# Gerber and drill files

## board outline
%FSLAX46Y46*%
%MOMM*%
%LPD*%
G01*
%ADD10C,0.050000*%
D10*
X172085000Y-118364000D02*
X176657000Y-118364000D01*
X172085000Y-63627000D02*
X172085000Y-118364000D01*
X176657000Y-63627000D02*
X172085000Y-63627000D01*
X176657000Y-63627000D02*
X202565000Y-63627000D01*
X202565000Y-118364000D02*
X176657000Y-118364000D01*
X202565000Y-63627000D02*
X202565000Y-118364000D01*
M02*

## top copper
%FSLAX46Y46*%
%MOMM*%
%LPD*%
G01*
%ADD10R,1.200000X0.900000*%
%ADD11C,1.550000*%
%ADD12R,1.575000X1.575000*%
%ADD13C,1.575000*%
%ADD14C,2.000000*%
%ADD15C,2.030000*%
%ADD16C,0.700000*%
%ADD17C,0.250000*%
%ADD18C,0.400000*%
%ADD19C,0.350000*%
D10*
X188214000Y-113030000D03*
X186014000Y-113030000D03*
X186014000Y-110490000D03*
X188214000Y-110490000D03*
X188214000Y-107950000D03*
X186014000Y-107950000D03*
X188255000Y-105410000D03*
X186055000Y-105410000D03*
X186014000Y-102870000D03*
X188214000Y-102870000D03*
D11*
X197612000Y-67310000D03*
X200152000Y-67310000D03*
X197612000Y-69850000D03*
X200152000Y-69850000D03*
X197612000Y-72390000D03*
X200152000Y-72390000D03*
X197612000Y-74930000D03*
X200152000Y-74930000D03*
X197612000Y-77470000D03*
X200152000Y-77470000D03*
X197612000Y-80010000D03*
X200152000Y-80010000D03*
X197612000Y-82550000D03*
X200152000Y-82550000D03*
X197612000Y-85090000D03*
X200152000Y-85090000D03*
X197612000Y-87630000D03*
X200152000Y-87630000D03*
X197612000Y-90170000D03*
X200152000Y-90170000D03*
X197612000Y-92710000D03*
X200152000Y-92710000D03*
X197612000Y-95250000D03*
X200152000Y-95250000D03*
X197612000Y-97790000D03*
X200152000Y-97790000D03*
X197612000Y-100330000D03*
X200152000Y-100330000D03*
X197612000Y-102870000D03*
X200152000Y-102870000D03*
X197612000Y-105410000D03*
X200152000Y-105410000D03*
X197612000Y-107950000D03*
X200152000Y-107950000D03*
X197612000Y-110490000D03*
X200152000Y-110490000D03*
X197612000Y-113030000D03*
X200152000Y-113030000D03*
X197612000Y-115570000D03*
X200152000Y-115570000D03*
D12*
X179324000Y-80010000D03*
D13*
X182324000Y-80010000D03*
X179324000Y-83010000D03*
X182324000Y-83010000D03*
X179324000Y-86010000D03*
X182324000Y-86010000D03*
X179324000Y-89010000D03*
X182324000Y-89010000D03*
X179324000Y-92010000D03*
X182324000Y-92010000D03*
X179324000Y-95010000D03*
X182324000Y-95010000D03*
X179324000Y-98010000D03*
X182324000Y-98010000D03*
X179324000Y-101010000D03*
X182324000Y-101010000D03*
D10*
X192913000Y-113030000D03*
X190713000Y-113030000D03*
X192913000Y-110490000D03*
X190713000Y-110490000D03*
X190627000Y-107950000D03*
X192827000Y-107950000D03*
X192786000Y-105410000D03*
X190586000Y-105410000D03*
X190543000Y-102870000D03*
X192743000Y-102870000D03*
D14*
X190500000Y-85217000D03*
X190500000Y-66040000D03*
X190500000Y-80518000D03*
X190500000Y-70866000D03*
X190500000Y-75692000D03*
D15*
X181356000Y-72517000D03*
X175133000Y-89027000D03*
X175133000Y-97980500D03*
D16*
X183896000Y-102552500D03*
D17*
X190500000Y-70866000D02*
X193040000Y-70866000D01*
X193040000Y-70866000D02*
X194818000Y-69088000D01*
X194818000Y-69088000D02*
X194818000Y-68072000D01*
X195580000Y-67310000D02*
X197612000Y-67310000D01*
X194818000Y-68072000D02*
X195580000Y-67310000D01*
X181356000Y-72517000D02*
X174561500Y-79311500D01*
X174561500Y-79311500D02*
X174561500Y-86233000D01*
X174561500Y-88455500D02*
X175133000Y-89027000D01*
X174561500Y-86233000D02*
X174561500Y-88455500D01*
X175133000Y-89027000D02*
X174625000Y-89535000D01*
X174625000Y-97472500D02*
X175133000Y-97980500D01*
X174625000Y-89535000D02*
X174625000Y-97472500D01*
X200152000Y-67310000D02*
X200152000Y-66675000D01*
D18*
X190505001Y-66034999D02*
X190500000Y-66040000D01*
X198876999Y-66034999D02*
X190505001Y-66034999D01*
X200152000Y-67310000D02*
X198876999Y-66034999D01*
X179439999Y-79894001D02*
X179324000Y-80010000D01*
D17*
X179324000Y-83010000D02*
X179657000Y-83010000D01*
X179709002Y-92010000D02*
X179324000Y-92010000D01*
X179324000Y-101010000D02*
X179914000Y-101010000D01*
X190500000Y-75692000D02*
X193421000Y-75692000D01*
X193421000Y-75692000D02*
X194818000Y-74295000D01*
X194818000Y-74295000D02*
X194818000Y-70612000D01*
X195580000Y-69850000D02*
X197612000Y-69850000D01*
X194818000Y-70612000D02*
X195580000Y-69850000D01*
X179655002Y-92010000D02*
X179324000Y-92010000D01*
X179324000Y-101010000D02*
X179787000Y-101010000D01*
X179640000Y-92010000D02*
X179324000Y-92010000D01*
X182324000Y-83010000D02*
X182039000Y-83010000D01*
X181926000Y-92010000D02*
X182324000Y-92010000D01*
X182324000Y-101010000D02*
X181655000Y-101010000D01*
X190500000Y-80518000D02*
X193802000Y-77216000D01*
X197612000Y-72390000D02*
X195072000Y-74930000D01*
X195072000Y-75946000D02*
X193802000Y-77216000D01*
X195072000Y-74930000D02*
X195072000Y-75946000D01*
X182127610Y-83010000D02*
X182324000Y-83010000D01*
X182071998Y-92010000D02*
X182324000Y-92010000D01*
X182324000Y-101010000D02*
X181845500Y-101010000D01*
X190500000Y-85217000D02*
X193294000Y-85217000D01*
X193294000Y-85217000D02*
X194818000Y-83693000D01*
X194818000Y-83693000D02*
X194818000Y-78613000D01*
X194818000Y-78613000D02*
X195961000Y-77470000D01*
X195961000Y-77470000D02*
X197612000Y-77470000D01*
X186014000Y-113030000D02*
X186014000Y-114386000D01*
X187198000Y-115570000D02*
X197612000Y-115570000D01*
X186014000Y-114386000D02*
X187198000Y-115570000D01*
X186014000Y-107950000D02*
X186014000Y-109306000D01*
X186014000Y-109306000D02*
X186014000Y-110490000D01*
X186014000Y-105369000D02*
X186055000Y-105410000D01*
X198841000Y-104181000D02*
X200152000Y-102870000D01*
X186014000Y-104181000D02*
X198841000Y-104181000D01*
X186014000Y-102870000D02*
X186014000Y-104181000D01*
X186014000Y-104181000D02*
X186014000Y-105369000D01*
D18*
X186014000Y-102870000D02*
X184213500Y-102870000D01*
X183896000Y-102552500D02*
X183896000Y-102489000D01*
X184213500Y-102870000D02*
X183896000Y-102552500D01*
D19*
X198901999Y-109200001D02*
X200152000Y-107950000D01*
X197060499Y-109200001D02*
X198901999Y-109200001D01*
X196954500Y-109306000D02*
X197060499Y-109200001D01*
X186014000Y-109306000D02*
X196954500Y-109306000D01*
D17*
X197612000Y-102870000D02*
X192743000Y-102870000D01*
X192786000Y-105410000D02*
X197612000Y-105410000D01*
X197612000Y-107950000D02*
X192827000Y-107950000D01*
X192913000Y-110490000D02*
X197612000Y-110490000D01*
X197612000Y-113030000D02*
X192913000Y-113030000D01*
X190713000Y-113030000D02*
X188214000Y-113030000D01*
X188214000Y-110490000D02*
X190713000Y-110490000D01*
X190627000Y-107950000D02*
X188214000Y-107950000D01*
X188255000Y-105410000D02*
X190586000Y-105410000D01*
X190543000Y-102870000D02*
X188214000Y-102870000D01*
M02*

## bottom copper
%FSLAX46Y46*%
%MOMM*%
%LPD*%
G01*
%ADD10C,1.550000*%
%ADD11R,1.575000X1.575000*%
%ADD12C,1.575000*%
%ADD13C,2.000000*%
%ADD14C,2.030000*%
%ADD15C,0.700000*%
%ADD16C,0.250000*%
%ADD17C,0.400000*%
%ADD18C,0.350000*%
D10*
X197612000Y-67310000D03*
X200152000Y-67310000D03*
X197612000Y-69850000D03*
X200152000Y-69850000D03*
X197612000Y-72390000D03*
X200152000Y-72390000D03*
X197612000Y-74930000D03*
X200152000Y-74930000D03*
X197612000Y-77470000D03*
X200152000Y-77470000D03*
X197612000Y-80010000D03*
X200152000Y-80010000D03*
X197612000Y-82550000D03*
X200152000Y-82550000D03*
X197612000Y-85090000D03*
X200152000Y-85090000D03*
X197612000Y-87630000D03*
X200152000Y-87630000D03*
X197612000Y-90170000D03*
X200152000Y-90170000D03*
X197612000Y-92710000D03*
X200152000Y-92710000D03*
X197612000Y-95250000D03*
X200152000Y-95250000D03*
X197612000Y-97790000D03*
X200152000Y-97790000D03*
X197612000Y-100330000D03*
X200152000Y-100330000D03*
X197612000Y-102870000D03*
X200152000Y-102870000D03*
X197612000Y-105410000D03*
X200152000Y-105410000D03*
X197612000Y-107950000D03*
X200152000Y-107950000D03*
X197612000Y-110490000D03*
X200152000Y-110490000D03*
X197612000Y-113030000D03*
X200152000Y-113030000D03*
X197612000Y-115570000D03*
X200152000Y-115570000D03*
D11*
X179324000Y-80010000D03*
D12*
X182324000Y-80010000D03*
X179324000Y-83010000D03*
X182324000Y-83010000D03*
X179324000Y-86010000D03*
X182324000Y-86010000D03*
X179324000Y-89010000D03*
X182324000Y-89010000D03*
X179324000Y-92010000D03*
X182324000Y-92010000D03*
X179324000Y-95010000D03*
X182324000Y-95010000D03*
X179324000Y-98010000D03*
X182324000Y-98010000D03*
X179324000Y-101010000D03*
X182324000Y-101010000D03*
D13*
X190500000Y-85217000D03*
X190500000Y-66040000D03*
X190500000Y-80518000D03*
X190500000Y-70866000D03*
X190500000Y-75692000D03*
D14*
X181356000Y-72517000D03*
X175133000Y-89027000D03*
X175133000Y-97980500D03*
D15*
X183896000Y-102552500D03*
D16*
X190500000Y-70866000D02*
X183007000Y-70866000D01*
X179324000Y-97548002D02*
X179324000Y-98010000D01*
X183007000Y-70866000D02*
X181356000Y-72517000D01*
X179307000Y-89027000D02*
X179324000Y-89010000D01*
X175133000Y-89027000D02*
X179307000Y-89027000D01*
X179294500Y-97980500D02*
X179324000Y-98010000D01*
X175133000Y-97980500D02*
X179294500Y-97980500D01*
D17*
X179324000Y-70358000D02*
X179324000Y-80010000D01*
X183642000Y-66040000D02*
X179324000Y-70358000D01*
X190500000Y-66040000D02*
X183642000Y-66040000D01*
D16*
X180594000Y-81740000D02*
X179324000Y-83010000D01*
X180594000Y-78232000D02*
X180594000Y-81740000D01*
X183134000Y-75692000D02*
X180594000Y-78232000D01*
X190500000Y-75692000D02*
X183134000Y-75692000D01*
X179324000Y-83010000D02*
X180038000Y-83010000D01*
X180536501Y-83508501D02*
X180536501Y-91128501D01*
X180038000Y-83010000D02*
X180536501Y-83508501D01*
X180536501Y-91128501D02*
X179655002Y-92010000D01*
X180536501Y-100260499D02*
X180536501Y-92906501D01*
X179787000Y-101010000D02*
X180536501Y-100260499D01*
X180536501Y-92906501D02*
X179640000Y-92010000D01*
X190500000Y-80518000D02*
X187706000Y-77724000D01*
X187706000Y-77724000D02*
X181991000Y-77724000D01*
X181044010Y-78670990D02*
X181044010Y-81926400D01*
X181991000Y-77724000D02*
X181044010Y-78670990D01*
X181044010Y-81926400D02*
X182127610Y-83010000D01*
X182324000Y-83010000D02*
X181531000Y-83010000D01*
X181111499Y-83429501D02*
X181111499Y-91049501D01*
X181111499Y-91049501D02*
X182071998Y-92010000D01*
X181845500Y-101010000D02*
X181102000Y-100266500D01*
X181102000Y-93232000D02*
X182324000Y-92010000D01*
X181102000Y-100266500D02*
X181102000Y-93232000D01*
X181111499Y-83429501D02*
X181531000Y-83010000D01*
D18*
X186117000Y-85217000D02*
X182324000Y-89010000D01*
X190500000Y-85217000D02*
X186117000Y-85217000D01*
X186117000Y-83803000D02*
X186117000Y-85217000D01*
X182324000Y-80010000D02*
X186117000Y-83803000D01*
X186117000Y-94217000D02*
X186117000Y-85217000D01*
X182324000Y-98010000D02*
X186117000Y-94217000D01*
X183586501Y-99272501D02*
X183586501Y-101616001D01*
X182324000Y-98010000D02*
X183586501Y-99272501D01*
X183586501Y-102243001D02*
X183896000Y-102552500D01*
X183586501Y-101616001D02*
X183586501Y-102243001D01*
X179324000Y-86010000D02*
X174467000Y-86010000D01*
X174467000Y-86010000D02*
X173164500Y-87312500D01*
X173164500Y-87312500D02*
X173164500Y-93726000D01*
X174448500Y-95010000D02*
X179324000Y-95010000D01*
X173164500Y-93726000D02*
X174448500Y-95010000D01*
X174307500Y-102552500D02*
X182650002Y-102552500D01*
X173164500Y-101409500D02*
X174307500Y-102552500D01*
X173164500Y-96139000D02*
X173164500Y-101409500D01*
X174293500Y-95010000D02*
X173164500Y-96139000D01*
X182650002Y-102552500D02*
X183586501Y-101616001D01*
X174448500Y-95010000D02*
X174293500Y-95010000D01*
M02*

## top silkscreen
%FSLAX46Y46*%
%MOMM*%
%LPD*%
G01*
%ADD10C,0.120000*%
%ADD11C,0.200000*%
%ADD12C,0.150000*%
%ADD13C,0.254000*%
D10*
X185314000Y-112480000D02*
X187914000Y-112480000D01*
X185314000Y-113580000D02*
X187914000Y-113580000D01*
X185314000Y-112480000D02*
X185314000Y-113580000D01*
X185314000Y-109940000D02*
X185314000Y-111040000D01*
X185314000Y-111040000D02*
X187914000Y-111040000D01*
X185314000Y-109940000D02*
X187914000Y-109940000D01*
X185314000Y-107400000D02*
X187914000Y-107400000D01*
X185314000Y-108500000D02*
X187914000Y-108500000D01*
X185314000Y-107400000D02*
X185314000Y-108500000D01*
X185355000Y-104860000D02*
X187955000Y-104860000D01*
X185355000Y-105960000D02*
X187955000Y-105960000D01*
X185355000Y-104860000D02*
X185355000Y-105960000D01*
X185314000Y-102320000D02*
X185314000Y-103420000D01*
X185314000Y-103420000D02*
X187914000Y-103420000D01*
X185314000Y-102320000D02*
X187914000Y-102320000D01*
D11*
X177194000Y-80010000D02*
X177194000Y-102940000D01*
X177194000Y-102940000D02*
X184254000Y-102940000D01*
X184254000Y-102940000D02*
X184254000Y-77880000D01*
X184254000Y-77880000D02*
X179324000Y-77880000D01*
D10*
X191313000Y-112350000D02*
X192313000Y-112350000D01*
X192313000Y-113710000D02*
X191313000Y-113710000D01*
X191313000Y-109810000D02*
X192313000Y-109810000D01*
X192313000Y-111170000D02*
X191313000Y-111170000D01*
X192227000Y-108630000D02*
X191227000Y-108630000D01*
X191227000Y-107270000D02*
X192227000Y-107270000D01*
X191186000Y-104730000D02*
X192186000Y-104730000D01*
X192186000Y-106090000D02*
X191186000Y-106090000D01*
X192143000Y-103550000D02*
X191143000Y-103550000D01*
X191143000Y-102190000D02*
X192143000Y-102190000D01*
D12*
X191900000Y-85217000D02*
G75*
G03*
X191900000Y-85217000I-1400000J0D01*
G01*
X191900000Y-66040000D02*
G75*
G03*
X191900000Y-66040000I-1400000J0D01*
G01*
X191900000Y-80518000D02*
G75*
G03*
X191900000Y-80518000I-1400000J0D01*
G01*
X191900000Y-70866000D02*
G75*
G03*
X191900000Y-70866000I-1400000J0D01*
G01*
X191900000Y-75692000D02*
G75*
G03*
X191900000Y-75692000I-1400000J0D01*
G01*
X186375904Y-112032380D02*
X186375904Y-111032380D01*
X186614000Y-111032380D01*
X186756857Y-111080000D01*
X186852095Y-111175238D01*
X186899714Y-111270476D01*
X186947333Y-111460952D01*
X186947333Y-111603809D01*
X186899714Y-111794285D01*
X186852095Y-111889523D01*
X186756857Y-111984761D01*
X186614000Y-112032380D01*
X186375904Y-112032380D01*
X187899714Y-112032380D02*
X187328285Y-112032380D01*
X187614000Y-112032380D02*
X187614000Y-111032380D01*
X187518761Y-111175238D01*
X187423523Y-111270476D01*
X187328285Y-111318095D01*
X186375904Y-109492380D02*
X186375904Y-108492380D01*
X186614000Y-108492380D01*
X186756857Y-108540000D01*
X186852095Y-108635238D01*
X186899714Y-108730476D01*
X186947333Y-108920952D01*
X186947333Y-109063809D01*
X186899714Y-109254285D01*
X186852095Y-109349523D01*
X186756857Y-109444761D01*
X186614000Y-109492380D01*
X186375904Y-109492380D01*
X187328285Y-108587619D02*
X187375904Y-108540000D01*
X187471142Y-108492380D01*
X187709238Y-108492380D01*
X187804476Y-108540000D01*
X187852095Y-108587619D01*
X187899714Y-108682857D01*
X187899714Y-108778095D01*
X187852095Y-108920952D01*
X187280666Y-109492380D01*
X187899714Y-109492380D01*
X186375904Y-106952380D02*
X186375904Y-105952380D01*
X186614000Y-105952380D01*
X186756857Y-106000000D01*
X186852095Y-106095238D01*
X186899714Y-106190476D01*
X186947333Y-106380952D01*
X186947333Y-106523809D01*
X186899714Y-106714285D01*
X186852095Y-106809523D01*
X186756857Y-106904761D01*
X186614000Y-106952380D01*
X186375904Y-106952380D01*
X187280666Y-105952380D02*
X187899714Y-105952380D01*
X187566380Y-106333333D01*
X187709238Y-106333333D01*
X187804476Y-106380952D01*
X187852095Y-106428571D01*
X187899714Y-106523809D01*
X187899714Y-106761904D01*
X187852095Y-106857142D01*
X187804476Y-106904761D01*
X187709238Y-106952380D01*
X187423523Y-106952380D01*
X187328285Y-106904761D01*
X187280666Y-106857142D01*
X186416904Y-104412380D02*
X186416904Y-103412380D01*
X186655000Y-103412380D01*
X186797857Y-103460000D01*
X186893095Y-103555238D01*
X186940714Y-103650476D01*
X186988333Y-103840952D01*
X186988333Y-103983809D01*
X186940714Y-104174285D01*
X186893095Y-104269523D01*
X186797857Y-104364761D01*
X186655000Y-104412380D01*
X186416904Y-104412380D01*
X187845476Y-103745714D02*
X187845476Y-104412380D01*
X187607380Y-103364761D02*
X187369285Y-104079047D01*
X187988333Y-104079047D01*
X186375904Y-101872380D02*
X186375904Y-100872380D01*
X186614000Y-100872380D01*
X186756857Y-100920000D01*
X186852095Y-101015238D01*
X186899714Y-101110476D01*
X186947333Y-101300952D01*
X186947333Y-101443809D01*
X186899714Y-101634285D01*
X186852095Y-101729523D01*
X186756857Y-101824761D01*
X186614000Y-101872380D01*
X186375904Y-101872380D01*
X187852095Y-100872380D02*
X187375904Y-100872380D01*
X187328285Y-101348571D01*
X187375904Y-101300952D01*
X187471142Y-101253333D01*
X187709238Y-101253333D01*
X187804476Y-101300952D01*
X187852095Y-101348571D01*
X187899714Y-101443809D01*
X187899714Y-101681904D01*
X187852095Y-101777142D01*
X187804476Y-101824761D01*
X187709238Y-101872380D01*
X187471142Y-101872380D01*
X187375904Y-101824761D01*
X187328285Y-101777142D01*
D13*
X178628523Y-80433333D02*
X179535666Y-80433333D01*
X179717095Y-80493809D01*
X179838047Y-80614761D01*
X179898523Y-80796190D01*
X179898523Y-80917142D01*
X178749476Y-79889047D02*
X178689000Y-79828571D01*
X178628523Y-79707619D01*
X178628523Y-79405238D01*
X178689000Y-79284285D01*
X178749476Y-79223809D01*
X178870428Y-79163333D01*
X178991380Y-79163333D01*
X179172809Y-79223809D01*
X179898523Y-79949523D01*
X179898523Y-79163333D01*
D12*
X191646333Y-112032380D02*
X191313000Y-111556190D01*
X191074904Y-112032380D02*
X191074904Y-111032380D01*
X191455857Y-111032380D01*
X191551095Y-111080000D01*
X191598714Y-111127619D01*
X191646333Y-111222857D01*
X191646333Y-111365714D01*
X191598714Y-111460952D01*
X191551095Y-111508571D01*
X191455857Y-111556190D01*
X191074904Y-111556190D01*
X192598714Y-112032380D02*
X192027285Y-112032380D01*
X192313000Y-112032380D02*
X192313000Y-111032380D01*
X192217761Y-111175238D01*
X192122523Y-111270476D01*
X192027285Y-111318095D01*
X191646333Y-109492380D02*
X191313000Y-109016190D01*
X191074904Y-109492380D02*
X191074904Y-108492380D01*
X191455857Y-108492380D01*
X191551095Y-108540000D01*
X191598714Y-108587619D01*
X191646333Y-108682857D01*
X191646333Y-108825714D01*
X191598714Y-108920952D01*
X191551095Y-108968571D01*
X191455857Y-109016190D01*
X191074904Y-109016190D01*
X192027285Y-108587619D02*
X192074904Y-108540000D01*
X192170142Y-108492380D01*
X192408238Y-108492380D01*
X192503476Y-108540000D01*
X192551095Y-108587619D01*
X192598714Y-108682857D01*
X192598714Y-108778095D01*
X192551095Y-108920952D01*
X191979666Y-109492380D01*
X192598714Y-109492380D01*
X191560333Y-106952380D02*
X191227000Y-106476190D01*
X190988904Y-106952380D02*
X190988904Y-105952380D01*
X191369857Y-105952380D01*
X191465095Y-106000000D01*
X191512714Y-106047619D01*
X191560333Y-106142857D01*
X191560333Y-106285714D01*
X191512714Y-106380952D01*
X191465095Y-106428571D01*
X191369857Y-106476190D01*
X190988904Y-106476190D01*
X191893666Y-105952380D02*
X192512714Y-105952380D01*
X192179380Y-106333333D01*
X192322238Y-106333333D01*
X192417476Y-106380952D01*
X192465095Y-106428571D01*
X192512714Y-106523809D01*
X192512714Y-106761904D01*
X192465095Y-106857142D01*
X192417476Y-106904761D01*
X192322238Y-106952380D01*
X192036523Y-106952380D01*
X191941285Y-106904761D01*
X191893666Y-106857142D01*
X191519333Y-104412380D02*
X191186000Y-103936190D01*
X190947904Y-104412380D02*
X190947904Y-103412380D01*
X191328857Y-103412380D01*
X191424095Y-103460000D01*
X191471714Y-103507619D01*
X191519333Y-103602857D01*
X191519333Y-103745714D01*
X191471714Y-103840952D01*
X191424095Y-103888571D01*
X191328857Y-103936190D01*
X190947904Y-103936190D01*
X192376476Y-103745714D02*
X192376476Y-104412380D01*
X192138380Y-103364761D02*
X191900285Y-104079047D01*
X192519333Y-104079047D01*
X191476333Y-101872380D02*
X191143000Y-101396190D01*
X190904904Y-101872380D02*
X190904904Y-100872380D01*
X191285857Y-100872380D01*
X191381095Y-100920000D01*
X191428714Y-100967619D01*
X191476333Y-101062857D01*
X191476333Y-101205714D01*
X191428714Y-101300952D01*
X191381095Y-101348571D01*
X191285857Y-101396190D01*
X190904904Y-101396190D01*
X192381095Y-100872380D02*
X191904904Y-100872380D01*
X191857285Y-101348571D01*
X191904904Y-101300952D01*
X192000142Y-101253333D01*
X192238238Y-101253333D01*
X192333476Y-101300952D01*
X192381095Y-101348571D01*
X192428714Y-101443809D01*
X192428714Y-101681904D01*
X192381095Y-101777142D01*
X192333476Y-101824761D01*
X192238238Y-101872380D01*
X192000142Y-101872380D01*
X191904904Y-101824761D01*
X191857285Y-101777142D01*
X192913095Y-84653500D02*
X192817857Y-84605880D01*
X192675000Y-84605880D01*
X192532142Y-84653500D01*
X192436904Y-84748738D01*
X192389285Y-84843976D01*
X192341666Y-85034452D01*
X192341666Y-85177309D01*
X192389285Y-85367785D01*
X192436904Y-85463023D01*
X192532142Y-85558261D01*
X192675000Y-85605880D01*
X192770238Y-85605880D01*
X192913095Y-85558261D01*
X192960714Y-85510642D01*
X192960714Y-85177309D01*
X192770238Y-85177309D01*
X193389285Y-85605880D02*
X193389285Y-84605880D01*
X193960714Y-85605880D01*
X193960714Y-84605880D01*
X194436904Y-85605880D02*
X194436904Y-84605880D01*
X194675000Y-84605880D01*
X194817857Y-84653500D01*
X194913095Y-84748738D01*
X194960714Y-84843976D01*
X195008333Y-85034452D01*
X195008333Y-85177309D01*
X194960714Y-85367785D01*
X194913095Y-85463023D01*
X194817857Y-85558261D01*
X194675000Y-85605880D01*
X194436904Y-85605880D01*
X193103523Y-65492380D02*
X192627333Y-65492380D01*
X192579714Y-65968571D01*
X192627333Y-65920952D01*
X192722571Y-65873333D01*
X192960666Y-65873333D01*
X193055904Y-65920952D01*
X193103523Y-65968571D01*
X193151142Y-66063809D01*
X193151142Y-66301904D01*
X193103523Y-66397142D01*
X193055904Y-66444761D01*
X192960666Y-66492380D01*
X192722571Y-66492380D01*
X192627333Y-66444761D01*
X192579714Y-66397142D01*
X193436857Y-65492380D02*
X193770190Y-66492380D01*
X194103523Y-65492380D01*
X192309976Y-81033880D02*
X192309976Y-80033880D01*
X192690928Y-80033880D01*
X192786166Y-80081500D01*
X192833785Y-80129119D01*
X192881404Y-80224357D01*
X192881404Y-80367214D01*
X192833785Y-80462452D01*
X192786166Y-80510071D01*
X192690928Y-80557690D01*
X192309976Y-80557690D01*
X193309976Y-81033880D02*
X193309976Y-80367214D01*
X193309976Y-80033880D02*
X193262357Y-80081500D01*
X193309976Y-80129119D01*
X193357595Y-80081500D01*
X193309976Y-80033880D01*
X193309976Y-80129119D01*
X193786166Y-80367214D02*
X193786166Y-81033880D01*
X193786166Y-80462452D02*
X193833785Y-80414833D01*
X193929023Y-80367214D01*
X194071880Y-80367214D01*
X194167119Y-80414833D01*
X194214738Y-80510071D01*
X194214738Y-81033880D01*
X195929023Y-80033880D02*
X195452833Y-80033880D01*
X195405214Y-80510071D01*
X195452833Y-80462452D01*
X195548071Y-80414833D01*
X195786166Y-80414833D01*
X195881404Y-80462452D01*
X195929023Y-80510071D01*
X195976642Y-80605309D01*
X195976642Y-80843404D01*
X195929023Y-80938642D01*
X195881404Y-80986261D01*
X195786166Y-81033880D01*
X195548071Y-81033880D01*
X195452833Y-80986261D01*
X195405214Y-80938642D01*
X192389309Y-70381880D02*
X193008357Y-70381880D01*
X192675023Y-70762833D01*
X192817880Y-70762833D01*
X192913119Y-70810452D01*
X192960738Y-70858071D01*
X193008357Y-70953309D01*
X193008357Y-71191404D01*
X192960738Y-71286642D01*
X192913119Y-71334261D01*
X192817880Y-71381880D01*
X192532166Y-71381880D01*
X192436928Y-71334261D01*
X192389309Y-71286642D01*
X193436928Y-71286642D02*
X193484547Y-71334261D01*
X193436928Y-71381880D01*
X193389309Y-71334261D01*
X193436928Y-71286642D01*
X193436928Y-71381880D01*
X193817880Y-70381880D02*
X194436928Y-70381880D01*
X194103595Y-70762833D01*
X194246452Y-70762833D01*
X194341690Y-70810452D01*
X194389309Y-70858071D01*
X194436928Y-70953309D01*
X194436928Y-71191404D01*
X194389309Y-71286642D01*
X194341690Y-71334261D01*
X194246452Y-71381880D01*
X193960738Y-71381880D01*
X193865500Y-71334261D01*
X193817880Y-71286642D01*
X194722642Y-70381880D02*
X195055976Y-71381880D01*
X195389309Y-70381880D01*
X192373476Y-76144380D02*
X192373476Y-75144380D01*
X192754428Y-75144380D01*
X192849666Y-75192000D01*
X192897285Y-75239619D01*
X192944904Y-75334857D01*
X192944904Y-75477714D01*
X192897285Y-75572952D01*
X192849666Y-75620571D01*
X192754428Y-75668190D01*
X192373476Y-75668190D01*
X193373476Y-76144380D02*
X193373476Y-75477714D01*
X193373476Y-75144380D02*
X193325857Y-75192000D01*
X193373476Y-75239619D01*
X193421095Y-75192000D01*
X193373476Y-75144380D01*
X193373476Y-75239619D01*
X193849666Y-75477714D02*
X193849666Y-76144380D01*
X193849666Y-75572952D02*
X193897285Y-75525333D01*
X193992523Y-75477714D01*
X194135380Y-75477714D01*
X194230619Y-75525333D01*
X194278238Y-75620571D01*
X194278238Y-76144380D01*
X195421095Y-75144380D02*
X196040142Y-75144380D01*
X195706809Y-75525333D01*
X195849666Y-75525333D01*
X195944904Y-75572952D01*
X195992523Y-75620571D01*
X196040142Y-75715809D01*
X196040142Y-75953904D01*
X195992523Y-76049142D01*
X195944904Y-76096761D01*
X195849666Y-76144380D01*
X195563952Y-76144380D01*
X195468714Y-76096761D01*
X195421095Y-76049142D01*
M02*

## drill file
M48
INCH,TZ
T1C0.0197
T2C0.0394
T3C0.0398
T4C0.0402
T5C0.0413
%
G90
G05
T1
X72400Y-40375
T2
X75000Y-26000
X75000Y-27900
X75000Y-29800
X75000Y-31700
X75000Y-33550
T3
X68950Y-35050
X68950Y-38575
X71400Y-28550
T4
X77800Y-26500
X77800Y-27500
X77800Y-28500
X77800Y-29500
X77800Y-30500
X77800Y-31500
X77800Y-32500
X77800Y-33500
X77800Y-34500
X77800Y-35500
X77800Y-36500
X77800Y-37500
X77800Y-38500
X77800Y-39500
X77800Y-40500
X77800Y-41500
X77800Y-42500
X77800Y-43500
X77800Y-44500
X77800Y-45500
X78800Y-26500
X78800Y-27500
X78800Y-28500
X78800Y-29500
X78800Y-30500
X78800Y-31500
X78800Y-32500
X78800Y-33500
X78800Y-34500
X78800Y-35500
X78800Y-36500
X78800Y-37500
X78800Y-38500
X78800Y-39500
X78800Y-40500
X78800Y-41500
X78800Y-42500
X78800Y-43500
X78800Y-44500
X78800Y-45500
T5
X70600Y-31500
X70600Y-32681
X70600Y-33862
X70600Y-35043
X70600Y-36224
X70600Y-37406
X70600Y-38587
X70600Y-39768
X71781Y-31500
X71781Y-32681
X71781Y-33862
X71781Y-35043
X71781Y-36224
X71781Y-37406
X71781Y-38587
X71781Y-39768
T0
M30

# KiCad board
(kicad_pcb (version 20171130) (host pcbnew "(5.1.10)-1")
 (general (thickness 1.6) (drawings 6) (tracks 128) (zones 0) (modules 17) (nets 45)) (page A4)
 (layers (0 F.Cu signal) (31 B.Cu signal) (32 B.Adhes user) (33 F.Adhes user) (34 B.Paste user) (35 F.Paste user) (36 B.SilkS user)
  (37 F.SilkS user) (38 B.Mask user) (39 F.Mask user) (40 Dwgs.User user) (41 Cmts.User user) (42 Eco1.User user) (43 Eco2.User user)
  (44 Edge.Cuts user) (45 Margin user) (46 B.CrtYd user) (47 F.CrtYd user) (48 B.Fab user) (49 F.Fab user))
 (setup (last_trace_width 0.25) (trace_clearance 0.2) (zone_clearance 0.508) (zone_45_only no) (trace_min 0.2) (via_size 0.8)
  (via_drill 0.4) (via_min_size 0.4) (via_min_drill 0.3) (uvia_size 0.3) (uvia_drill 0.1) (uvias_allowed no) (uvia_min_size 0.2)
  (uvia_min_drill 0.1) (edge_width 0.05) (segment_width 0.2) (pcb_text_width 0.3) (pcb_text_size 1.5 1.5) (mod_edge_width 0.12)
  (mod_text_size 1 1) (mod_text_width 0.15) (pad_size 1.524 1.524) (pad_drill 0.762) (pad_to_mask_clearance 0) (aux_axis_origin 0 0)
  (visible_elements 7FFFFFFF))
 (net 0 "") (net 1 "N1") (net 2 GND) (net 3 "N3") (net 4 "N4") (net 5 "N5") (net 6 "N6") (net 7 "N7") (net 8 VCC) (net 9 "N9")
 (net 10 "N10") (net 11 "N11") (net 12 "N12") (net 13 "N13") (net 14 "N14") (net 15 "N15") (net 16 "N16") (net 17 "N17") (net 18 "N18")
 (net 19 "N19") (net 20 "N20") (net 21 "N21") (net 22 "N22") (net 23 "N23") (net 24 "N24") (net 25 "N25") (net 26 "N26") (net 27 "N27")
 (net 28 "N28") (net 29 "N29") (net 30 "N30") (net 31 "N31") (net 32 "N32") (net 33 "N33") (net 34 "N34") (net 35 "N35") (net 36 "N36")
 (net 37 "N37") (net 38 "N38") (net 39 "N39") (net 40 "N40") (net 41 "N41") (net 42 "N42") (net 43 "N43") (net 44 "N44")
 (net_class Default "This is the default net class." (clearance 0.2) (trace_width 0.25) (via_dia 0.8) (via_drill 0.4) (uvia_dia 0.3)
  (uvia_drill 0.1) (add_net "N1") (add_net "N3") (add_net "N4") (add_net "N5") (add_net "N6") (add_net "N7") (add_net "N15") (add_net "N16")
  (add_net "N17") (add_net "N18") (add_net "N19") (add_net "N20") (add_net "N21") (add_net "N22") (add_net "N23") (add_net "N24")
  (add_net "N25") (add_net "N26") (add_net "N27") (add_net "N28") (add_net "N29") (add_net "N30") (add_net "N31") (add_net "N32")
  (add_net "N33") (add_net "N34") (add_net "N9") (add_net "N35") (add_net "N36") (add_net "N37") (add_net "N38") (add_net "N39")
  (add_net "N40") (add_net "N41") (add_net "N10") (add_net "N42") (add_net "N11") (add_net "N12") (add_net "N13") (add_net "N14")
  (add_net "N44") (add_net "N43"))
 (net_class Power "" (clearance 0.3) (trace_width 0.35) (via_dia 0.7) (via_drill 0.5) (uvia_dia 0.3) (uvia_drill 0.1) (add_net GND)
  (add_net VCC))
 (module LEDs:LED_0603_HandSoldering (layer F.Cu) (at 187.114 113.03)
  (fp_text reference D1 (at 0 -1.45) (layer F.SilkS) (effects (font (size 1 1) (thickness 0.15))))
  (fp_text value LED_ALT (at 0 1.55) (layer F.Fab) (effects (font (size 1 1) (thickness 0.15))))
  (fp_line (start -1.8 -0.55) (end 0.8 -0.55) (layer F.SilkS) (width 0.12))
  (fp_line (start -1.8 0.55) (end 0.8 0.55) (layer F.SilkS) (width 0.12))
  (fp_line (start -1.8 -0.55) (end -1.8 0.55) (layer F.SilkS) (width 0.12))
  (pad 2 smd rect (at 1.1 0) (size 1.2 0.9) (layers F.Cu F.Paste F.Mask) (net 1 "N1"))
  (pad 1 smd rect (at -1.1 0) (size 1.2 0.9) (layers F.Cu F.Paste F.Mask) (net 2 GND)))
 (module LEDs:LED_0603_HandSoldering (layer F.Cu) (at 187.114 110.49)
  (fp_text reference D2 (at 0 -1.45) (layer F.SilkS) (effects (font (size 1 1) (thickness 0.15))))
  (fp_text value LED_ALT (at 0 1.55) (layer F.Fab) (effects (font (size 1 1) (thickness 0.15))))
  (fp_line (start -1.8 -0.55) (end -1.8 0.55) (layer F.SilkS) (width 0.12))
  (fp_line (start -1.8 0.55) (end 0.8 0.55) (layer F.SilkS) (width 0.12))
  (fp_line (start -1.8 -0.55) (end 0.8 -0.55) (layer F.SilkS) (width 0.12))
  (pad 1 smd rect (at -1.1 0) (size 1.2 0.9) (layers F.Cu F.Paste F.Mask) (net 2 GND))
  (pad 2 smd rect (at 1.1 0) (size 1.2 0.9) (layers F.Cu F.Paste F.Mask) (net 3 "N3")))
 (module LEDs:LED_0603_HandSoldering (layer F.Cu) (at 187.114 107.95)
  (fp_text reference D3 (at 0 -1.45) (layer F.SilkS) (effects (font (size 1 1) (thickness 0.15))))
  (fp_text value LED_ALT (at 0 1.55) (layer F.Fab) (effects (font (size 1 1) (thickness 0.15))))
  (fp_line (start -1.8 -0.55) (end 0.8 -0.55) (layer F.SilkS) (width 0.12))
  (fp_line (start -1.8 0.55) (end 0.8 0.55) (layer F.SilkS) (width 0.12))
  (fp_line (start -1.8 -0.55) (end -1.8 0.55) (layer F.SilkS) (width 0.12))
  (pad 2 smd rect (at 1.1 0) (size 1.2 0.9) (layers F.Cu F.Paste F.Mask) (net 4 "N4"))
  (pad 1 smd rect (at -1.1 0) (size 1.2 0.9) (layers F.Cu F.Paste F.Mask) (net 2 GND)))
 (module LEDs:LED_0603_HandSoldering (layer F.Cu) (at 187.155 105.41)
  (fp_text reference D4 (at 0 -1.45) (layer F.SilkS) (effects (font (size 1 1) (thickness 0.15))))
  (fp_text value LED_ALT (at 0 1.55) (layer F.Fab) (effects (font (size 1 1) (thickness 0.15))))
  (fp_line (start -1.8 -0.55) (end 0.8 -0.55) (layer F.SilkS) (width 0.12))
  (fp_line (start -1.8 0.55) (end 0.8 0.55) (layer F.SilkS) (width 0.12))
  (fp_line (start -1.8 -0.55) (end -1.8 0.55) (layer F.SilkS) (width 0.12))
  (pad 2 smd rect (at 1.1 0) (size 1.2 0.9) (layers F.Cu F.Paste F.Mask) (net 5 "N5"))
  (pad 1 smd rect (at -1.1 0) (size 1.2 0.9) (layers F.Cu F.Paste F.Mask) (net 2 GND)))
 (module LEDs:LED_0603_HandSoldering (layer F.Cu) (at 187.114 102.87)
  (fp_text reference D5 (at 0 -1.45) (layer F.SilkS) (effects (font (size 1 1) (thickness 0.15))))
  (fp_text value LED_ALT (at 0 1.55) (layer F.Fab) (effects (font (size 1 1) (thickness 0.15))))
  (fp_line (start -1.8 -0.55) (end -1.8 0.55) (layer F.SilkS) (width 0.12))
  (fp_line (start -1.8 0.55) (end 0.8 0.55) (layer F.SilkS) (width 0.12))
  (fp_line (start -1.8 -0.55) (end 0.8 -0.55) (layer F.SilkS) (width 0.12))
  (pad 1 smd rect (at -1.1 0) (size 1.2 0.9) (layers F.Cu F.Paste F.Mask) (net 2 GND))
  (pad 2 smd rect (at 1.1 0) (size 1.2 0.9) (layers F.Cu F.Paste F.Mask) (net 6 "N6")))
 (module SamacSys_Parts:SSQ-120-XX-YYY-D (layer B.Cu) (at 197.612 67.31 90)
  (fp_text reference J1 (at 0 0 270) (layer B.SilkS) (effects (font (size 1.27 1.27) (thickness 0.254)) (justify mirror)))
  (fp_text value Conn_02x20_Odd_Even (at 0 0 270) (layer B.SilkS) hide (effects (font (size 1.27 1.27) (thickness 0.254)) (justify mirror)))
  (pad 1 thru_hole circle (at 0 0 90) (size 1.55 1.55) (drill 1.02) (layers *.Cu *.Mask) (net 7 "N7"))
  (pad 2 thru_hole circle (at 0 2.54 90) (size 1.55 1.55) (drill 1.02) (layers *.Cu *.Mask) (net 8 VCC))
  (pad 3 thru_hole circle (at -2.54 0 90) (size 1.55 1.55) (drill 1.02) (layers *.Cu *.Mask) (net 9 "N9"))
  (pad 4 thru_hole circle (at -2.54 2.54 90) (size 1.55 1.55) (drill 1.02) (layers *.Cu *.Mask) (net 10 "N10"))
  (pad 5 thru_hole circle (at -5.08 0 90) (size 1.55 1.55) (drill 1.02) (layers *.Cu *.Mask) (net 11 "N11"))
  (pad 6 thru_hole circle (at -5.08 2.54 90) (size 1.55 1.55) (drill 1.02) (layers *.Cu *.Mask) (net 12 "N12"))
  (pad 7 thru_hole circle (at -7.62 0 90) (size 1.55 1.55) (drill 1.02) (layers *.Cu *.Mask) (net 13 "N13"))
  (pad 8 thru_hole circle (at -7.62 2.54 90) (size 1.55 1.55) (drill 1.02) (layers *.Cu *.Mask) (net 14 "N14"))
  (pad 9 thru_hole circle (at -10.16 0 90) (size 1.55 1.55) (drill 1.02) (layers *.Cu *.Mask) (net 2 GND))
  (pad 10 thru_hole circle (at -10.16 2.54 90) (size 1.55 1.55) (drill 1.02) (layers *.Cu *.Mask) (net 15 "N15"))
  (pad 11 thru_hole circle (at -12.7 0 90) (size 1.55 1.55) (drill 1.02) (layers *.Cu *.Mask) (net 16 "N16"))
  (pad 12 thru_hole circle (at -12.7 2.54 90) (size 1.55 1.55) (drill 1.02) (layers *.Cu *.Mask) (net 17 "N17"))
  (pad 13 thru_hole circle (at -15.24 0 90) (size 1.55 1.55) (drill 1.02) (layers *.Cu *.Mask) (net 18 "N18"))
  (pad 14 thru_hole circle (at -15.24 2.54 90) (size 1.55 1.55) (drill 1.02) (layers *.Cu *.Mask) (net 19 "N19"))
  (pad 15 thru_hole circle (at -17.78 0 90) (size 1.55 1.55) (drill 1.02) (layers *.Cu *.Mask) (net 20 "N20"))
  (pad 16 thru_hole circle (at -17.78 2.54 90) (size 1.55 1.55) (drill 1.02) (layers *.Cu *.Mask) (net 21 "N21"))
  (pad 17 thru_hole circle (at -20.32 0 90) (size 1.55 1.55) (drill 1.02) (layers *.Cu *.Mask) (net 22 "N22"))
  (pad 18 thru_hole circle (at -20.32 2.54 90) (size 1.55 1.55) (drill 1.02) (layers *.Cu *.Mask) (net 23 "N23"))
  (pad 19 thru_hole circle (at -22.86 0 90) (size 1.55 1.55) (drill 1.02) (layers *.Cu *.Mask) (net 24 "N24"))
  (pad 20 thru_hole circle (at -22.86 2.54 90) (size 1.55 1.55) (drill 1.02) (layers *.Cu *.Mask) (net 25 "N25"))
  (pad 21 thru_hole circle (at -25.4 0 90) (size 1.55 1.55) (drill 1.02) (layers *.Cu *.Mask) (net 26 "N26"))
  (pad 22 thru_hole circle (at -25.4 2.54 90) (size 1.55 1.55) (drill 1.02) (layers *.Cu *.Mask) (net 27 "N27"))
  (pad 23 thru_hole circle (at -27.94 0 90) (size 1.55 1.55) (drill 1.02) (layers *.Cu *.Mask) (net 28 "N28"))
  (pad 24 thru_hole circle (at -27.94 2.54 90) (size 1.55 1.55) (drill 1.02) (layers *.Cu *.Mask) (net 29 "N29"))
  (pad 25 thru_hole circle (at -30.48 0 90) (size 1.55 1.55) (drill 1.02) (layers *.Cu *.Mask) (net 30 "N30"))
  (pad 26 thru_hole circle (at -30.48 2.54 90) (size 1.55 1.55) (drill 1.02) (layers *.Cu *.Mask) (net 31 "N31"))
  (pad 27 thru_hole circle (at -33.02 0 90) (size 1.55 1.55) (drill 1.02) (layers *.Cu *.Mask) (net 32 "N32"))
  (pad 28 thru_hole circle (at -33.02 2.54 90) (size 1.55 1.55) (drill 1.02) (layers *.Cu *.Mask) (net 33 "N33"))
  (pad 29 thru_hole circle (at -35.56 0 90) (size 1.55 1.55) (drill 1.02) (layers *.Cu *.Mask) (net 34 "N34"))
  (pad 30 thru_hole circle (at -35.56 2.54 90) (size 1.55 1.55) (drill 1.02) (layers *.Cu *.Mask) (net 2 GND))
  (pad 31 thru_hole circle (at -38.1 0 90) (size 1.55 1.55) (drill 1.02) (layers *.Cu *.Mask) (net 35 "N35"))
  (pad 32 thru_hole circle (at -38.1 2.54 90) (size 1.55 1.55) (drill 1.02) (layers *.Cu *.Mask) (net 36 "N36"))
  (pad 33 thru_hole circle (at -40.64 0 90) (size 1.55 1.55) (drill 1.02) (layers *.Cu *.Mask) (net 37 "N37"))
  (pad 34 thru_hole circle (at -40.64 2.54 90) (size 1.55 1.55) (drill 1.02) (layers *.Cu *.Mask) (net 2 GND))
  (pad 35 thru_hole circle (at -43.18 0 90) (size 1.55 1.55) (drill 1.02) (layers *.Cu *.Mask) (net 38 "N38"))
  (pad 36 thru_hole circle (at -43.18 2.54 90) (size 1.55 1.55) (drill 1.02) (layers *.Cu *.Mask) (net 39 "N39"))
  (pad 37 thru_hole circle (at -45.72 0 90) (size 1.55 1.55) (drill 1.02) (layers *.Cu *.Mask) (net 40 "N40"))
  (pad 38 thru_hole circle (at -45.72 2.54 90) (size 1.55 1.55) (drill 1.02) (layers *.Cu *.Mask) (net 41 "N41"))
  (pad 39 thru_hole circle (at -48.26 0 90) (size 1.55 1.55) (drill 1.02) (layers *.Cu *.Mask) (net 2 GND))
  (pad 40 thru_hole circle (at -48.26 2.54 90) (size 1.55 1.55) (drill 1.02) (layers *.Cu *.Mask) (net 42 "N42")))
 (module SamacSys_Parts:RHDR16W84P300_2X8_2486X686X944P (layer F.Cu) (at 179.324 80.01 90)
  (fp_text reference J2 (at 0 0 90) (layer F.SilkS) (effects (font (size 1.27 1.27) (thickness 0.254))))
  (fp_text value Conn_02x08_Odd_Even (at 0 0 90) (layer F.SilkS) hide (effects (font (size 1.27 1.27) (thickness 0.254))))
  (fp_line (start 0 -2.13) (end -22.93 -2.13) (layer F.SilkS) (width 0.2))
  (fp_line (start -22.93 -2.13) (end -22.93 4.93) (layer F.SilkS) (width 0.2))
  (fp_line (start -22.93 4.93) (end 2.13 4.93) (layer F.SilkS) (width 0.2))
  (fp_line (start 2.13 4.93) (end 2.13 0) (layer F.SilkS) (width 0.2))
  (pad 1 thru_hole rect (at 0 0 90) (size 1.575 1.575) (drill 1.05) (layers *.Cu *.Mask) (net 8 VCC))
  (pad 2 thru_hole circle (at 0 3 90) (size 1.575 1.575) (drill 1.05) (layers *.Cu *.Mask) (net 2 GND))
  (pad 3 thru_hole circle (at -3 0 90) (size 1.575 1.575) (drill 1.05) (layers *.Cu *.Mask) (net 9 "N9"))
  (pad 4 thru_hole circle (at -3 3 90) (size 1.575 1.575) (drill 1.05) (layers *.Cu *.Mask) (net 11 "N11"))
  (pad 5 thru_hole circle (at -6 0 90) (size 1.575 1.575) (drill 1.05) (layers *.Cu *.Mask) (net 2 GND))
  (pad 6 thru_hole circle (at -6 3 90) (size 1.575 1.575) (drill 1.05) (layers *.Cu *.Mask) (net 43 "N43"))
  (pad 7 thru_hole circle (at -9 0 90) (size 1.575 1.575) (drill 1.05) (layers *.Cu *.Mask) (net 7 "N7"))
  (pad 8 thru_hole circle (at -9 3 90) (size 1.575 1.575) (drill 1.05) (layers *.Cu *.Mask) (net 2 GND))
  (pad 9 thru_hole circle (at -12 0 90) (size 1.575 1.575) (drill 1.05) (layers *.Cu *.Mask) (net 9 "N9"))
  (pad 10 thru_hole circle (at -12 3 90) (size 1.575 1.575) (drill 1.05) (layers *.Cu *.Mask) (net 11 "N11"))
  (pad 11 thru_hole circle (at -15 0 90) (size 1.575 1.575) (drill 1.05) (layers *.Cu *.Mask) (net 2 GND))
  (pad 12 thru_hole circle (at -15 3 90) (size 1.575 1.575) (drill 1.05) (layers *.Cu *.Mask) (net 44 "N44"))
  (pad 13 thru_hole circle (at -18 0 90) (size 1.575 1.575) (drill 1.05) (layers *.Cu *.Mask) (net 7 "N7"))
  (pad 14 thru_hole circle (at -18 3 90) (size 1.575 1.575) (drill 1.05) (layers *.Cu *.Mask) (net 2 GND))
  (pad 15 thru_hole circle (at -21 0 90) (size 1.575 1.575) (drill 1.05) (layers *.Cu *.Mask) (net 9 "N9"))
  (pad 16 thru_hole circle (at -21 3 90) (size 1.575 1.575) (drill 1.05) (layers *.Cu *.Mask) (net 11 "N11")))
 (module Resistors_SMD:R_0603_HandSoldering (layer F.Cu) (at 191.813 113.03)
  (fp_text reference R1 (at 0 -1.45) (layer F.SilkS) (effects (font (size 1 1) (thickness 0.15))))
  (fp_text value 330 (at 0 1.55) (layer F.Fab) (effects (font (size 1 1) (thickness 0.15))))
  (fp_line (start -0.5 -0.68) (end 0.5 -0.68) (layer F.SilkS) (width 0.12))
  (fp_line (start 0.5 0.68) (end -0.5 0.68) (layer F.SilkS) (width 0.12))
  (pad 2 smd rect (at 1.1 0) (size 1.2 0.9) (layers F.Cu F.Paste F.Mask) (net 40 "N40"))
  (pad 1 smd rect (at -1.1 0) (size 1.2 0.9) (layers F.Cu F.Paste F.Mask) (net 1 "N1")))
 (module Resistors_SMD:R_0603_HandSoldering (layer F.Cu) (at 191.813 110.49)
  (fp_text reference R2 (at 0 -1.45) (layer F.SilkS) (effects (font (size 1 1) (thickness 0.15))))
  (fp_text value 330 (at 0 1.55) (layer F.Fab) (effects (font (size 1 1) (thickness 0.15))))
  (fp_line (start -0.5 -0.68) (end 0.5 -0.68) (layer F.SilkS) (width 0.12))
  (fp_line (start 0.5 0.68) (end -0.5 0.68) (layer F.SilkS) (width 0.12))
  (pad 2 smd rect (at 1.1 0) (size 1.2 0.9) (layers F.Cu F.Paste F.Mask) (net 38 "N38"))
  (pad 1 smd rect (at -1.1 0) (size 1.2 0.9) (layers F.Cu F.Paste F.Mask) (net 3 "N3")))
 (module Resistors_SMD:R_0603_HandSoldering (layer F.Cu) (at 191.727 107.95)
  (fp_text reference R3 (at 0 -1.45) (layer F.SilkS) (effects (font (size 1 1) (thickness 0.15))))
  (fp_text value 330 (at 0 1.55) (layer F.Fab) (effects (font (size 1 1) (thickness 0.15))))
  (fp_line (start 0.5 0.68) (end -0.5 0.68) (layer F.SilkS) (width 0.12))
  (fp_line (start -0.5 -0.68) (end 0.5 -0.68) (layer F.SilkS) (width 0.12))
  (pad 1 smd rect (at -1.1 0) (size 1.2 0.9) (layers F.Cu F.Paste F.Mask) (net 4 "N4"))
  (pad 2 smd rect (at 1.1 0) (size 1.2 0.9) (layers F.Cu F.Paste F.Mask) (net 37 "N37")))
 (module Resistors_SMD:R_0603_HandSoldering (layer F.Cu) (at 191.686 105.41)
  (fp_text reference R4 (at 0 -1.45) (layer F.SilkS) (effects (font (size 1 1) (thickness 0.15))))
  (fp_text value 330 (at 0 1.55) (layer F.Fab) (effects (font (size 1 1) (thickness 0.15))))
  (fp_line (start -0.5 -0.68) (end 0.5 -0.68) (layer F.SilkS) (width 0.12))
  (fp_line (start 0.5 0.68) (end -0.5 0.68) (layer F.SilkS) (width 0.12))
  (pad 2 smd rect (at 1.1 0) (size 1.2 0.9) (layers F.Cu F.Paste F.Mask) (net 35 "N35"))
  (pad 1 smd rect (at -1.1 0) (size 1.2 0.9) (layers F.Cu F.Paste F.Mask) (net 5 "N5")))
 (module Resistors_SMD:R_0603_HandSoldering (layer F.Cu) (at 191.643 102.87)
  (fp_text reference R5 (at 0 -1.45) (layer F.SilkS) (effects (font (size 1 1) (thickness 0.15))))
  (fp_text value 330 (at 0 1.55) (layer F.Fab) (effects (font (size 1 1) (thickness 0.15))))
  (fp_line (start 0.5 0.68) (end -0.5 0.68) (layer F.SilkS) (width 0.12))
  (fp_line (start -0.5 -0.68) (end 0.5 -0.68) (layer F.SilkS) (width 0.12))
  (pad 1 smd rect (at -1.1 0) (size 1.2 0.9) (layers F.Cu F.Paste F.Mask) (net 6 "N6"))
  (pad 2 smd rect (at 1.1 0) (size 1.2 0.9) (layers F.Cu F.Paste F.Mask) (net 34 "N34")))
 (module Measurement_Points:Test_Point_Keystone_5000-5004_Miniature (layer F.Cu) (at 190.5 85.217)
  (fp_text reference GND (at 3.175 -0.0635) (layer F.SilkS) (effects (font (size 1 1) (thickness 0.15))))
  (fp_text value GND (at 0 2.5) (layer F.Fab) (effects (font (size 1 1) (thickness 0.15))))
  (fp_circle (center 0 0) (end 1.4 0) (layer F.SilkS) (width 0.15))
  (pad 1 thru_hole circle (at 0 0) (size 2 2) (drill 1) (layers *.Cu *.Mask) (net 2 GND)))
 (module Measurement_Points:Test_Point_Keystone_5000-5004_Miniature (layer F.Cu) (at 190.5 66.04)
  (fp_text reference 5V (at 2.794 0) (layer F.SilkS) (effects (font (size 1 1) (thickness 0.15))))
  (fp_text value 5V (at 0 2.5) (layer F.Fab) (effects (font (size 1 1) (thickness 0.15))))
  (fp_circle (center 0 0) (end 1.4 0) (layer F.SilkS) (width 0.15))
  (pad 1 thru_hole circle (at 0 0) (size 2 2) (drill 1) (layers *.Cu *.Mask) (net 8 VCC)))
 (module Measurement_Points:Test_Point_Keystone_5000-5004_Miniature (layer F.Cu) (at 190.5 80.518)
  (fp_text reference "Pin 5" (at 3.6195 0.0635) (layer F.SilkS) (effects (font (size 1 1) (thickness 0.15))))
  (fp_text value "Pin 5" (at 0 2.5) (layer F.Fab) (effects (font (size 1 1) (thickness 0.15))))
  (fp_circle (center 0 0) (end 1.4 0) (layer F.SilkS) (width 0.15))
  (pad 1 thru_hole circle (at 0 0) (size 2 2) (drill 1) (layers *.Cu *.Mask) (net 11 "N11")))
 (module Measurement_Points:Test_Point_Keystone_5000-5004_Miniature (layer F.Cu) (at 190.5 70.866)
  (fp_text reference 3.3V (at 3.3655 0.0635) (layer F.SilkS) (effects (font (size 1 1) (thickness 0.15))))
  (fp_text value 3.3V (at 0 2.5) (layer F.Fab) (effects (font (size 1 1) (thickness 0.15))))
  (fp_circle (center 0 0) (end 1.4 0) (layer F.SilkS) (width 0.15))
  (pad 1 thru_hole circle (at 0 0) (size 2 2) (drill 1) (layers *.Cu *.Mask) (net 7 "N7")))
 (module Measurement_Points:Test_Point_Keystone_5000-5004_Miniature (layer F.Cu) (at 190.5 75.692)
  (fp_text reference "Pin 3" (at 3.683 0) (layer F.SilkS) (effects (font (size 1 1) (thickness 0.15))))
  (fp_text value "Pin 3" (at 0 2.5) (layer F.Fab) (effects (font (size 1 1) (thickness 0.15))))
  (fp_circle (center 0 0) (end 1.4 0) (layer F.SilkS) (width 0.15))
  (pad 1 thru_hole circle (at 0 0) (size 2 2) (drill 1) (layers *.Cu *.Mask) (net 9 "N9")))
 (gr_line (start 172.085 118.364) (end 176.657 118.364) (layer Edge.Cuts) (width 0.05))
 (gr_line (start 172.085 63.627) (end 172.085 118.364) (layer Edge.Cuts) (width 0.05))
 (gr_line (start 176.657 63.627) (end 172.085 63.627) (layer Edge.Cuts) (width 0.05))
 (gr_line (start 176.657 63.627) (end 202.565 63.627) (layer Edge.Cuts) (width 0.05))
 (gr_line (start 202.565 118.364) (end 176.657 118.364) (layer Edge.Cuts) (width 0.05))
 (gr_line (start 202.565 63.627) (end 202.565 118.364) (layer Edge.Cuts) (width 0.05))
 (segment (start 190.5 70.866) (end 193.04 70.866) (width 0.25) (layer F.Cu) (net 7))
 (segment (start 193.04 70.866) (end 194.818 69.088) (width 0.25) (layer F.Cu) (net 7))
 (segment (start 194.818 69.088) (end 194.818 68.072) (width 0.25) (layer F.Cu) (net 7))
 (segment (start 195.58 67.31) (end 197.612 67.31) (width 0.25) (layer F.Cu) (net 7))
 (segment (start 194.818 68.072) (end 195.58 67.31) (width 0.25) (layer F.Cu) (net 7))
 (segment (start 190.5 70.866) (end 183.007 70.866) (width 0.25) (layer B.Cu) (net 7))
 (segment (start 179.324 97.548002) (end 179.324 98.01) (width 0.25) (layer B.Cu) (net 7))
 (via (at 181.356 72.517) (size 2.03) (drill 1.01) (layers F.Cu B.Cu) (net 7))
 (segment (start 183.007 70.866) (end 181.356 72.517) (width 0.25) (layer B.Cu) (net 7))
 (segment (start 181.356 72.517) (end 174.5615 79.3115) (width 0.25) (layer F.Cu) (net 7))
 (segment (start 174.5615 79.3115) (end 174.5615 86.233) (width 0.25) (layer F.Cu) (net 7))
 (via (at 175.133 89.027) (size 2.03) (drill 1.01) (layers F.Cu B.Cu) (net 7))
 (segment (start 174.5615 88.4555) (end 175.133 89.027) (width 0.25) (layer F.Cu) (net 7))
 (segment (start 174.5615 86.233) (end 174.5615 88.4555) (width 0.25) (layer F.Cu) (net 7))
 (segment (start 179.307 89.027) (end 179.324 89.01) (width 0.25) (layer B.Cu) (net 7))
 (segment (start 175.133 89.027) (end 179.307 89.027) (width 0.25) (layer B.Cu) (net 7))
 (segment (start 175.133 89.027) (end 174.625 89.535) (width 0.25) (layer F.Cu) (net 7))
 (via (at 175.133 97.9805) (size 2.03) (drill 1.01) (layers F.Cu B.Cu) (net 7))
 (segment (start 174.625 97.4725) (end 175.133 97.9805) (width 0.25) (layer F.Cu) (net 7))
 (segment (start 174.625 89.535) (end 174.625 97.4725) (width 0.25) (layer F.Cu) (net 7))
 (segment (start 179.2945 97.9805) (end 179.324 98.01) (width 0.25) (layer B.Cu) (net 7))
 (segment (start 175.133 97.9805) (end 179.2945 97.9805) (width 0.25) (layer B.Cu) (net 7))
 (segment (start 200.152 67.31) (end 200.152 66.675) (width 0.25) (layer F.Cu) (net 8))
 (segment (start 190.505001 66.034999) (end 190.5 66.04) (width 0.4) (layer F.Cu) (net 8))
 (segment (start 198.876999 66.034999) (end 190.505001 66.034999) (width 0.4) (layer F.Cu) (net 8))
 (segment (start 200.152 67.31) (end 198.876999 66.034999) (width 0.4) (layer F.Cu) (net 8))
 (segment (start 179.439999 79.894001) (end 179.324 80.01) (width 0.4) (layer F.Cu) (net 8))
 (segment (start 179.324 70.358) (end 179.324 80.01) (width 0.4) (layer B.Cu) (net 8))
 (segment (start 183.642 66.04) (end 179.324 70.358) (width 0.4) (layer B.Cu) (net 8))
 (segment (start 190.5 66.04) (end 183.642 66.04) (width 0.4) (layer B.Cu) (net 8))
 (segment (start 179.324 83.01) (end 179.657 83.01) (width 0.25) (layer F.Cu) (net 9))
 (segment (start 179.709002 92.01) (end 179.324 92.01) (width 0.25) (layer F.Cu) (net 9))
 (segment (start 179.324 101.01) (end 179.914 101.01) (width 0.25) (layer F.Cu) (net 9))
 (segment (start 190.5 75.692) (end 193.421 75.692) (width 0.25) (layer F.Cu) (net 9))
 (segment (start 193.421 75.692) (end 194.818 74.295) (width 0.25) (layer F.Cu) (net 9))
 (segment (start 194.818 74.295) (end 194.818 70.612) (width 0.25) (layer F.Cu) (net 9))
 (segment (start 195.58 69.85) (end 197.612 69.85) (width 0.25) (layer F.Cu) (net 9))
 (segment (start 194.818 70.612) (end 195.58 69.85) (width 0.25) (layer F.Cu) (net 9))
 (segment (start 180.594 81.74) (end 179.324 83.01) (width 0.25) (layer B.Cu) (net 9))
 (segment (start 180.594 78.232) (end 180.594 81.74) (width 0.25) (layer B.Cu) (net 9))
 (segment (start 183.134 75.692) (end 180.594 78.232) (width 0.25) (layer B.Cu) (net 9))
 (segment (start 190.5 75.692) (end 183.134 75.692) (width 0.25) (layer B.Cu) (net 9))
 (segment (start 179.324 83.01) (end 180.038 83.01) (width 0.25) (layer B.Cu) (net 9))
 (segment (start 180.536501 83.508501) (end 180.536501 91.128501) (width 0.25) (layer B.Cu) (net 9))
 (segment (start 180.038 83.01) (end 180.536501 83.508501) (width 0.25) (layer B.Cu) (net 9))
 (segment (start 179.655002 92.01) (end 179.324 92.01) (width 0.25) (layer F.Cu) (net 9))
 (segment (start 180.536501 91.128501) (end 179.655002 92.01) (width 0.25) (layer B.Cu) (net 9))
 (segment (start 179.324 101.01) (end 179.787 101.01) (width 0.25) (layer F.Cu) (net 9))
 (segment (start 180.536501 100.260499) (end 180.536501 92.906501) (width 0.25) (layer B.Cu) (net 9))
 (segment (start 179.787 101.01) (end 180.536501 100.260499) (width 0.25) (layer B.Cu) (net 9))
 (segment (start 179.64 92.01) (end 179.324 92.01) (width 0.25) (layer F.Cu) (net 9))
 (segment (start 180.536501 92.906501) (end 179.64 92.01) (width 0.25) (layer B.Cu) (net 9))
 (segment (start 182.324 83.01) (end 182.039 83.01) (width 0.25) (layer F.Cu) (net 11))
 (segment (start 181.926 92.01) (end 182.324 92.01) (width 0.25) (layer F.Cu) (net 11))
 (segment (start 182.324 101.01) (end 181.655 101.01) (width 0.25) (layer F.Cu) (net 11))
 (segment (start 190.5 80.518) (end 193.802 77.216) (width 0.25) (layer F.Cu) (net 11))
 (segment (start 197.612 72.39) (end 195.072 74.93) (width 0.25) (layer F.Cu) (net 11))
 (segment (start 195.072 75.946) (end 193.802 77.216) (width 0.25) (layer F.Cu) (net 11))
 (segment (start 195.072 74.93) (end 195.072 75.946) (width 0.25) (layer F.Cu) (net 11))
 (segment (start 190.5 80.518) (end 187.706 77.724) (width 0.25) (layer B.Cu) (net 11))
 (segment (start 187.706 77.724) (end 181.991 77.724) (width 0.25) (layer B.Cu) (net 11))
 (segment (start 181.04401 78.67099) (end 181.04401 81.9264) (width 0.25) (layer B.Cu) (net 11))
 (segment (start 181.991 77.724) (end 181.04401 78.67099) (width 0.25) (layer B.Cu) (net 11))
 (segment (start 182.12761 83.01) (end 182.324 83.01) (width 0.25) (layer F.Cu) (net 11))
 (segment (start 181.04401 81.9264) (end 182.12761 83.01) (width 0.25) (layer B.Cu) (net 11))
 (segment (start 182.324 83.01) (end 181.531 83.01) (width 0.25) (layer B.Cu) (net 11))
 (segment (start 181.111499 83.429501) (end 181.111499 91.049501) (width 0.25) (layer B.Cu) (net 11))
 (segment (start 182.071998 92.01) (end 182.324 92.01) (width 0.25) (layer F.Cu) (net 11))
 (segment (start 181.111499 91.049501) (end 182.071998 92.01) (width 0.25) (layer B.Cu) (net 11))
 (segment (start 182.324 101.01) (end 181.8455 101.01) (width 0.25) (layer F.Cu) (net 11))
 (segment (start 181.8455 101.01) (end 181.102 100.2665) (width 0.25) (layer B.Cu) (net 11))
 (segment (start 181.102 93.232) (end 182.324 92.01) (width 0.25) (layer B.Cu) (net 11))
 (segment (start 181.102 100.2665) (end 181.102 93.232) (width 0.25) (layer B.Cu) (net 11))
 (segment (start 181.111499 83.429501) (end 181.531 83.01) (width 0.25) (layer B.Cu) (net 11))
 (segment (start 190.5 85.217) (end 193.294 85.217) (width 0.25) (layer F.Cu) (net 2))
 (segment (start 193.294 85.217) (end 194.818 83.693) (width 0.25) (layer F.Cu) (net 2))
 (segment (start 194.818 83.693) (end 194.818 78.613) (width 0.25) (layer F.Cu) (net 2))
 (segment (start 194.818 78.613) (end 195.961 77.47) (width 0.25) (layer F.Cu) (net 2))
 (segment (start 195.961 77.47) (end 197.612 77.47) (width 0.25) (layer F.Cu) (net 2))
 (segment (start 186.014 113.03) (end 186.014 114.386) (width 0.25) (layer F.Cu) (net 2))
 (segment (start 187.198 115.57) (end 197.612 115.57) (width 0.25) (layer F.Cu) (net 2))
 (segment (start 186.014 114.386) (end 187.198 115.57) (width 0.25) (layer F.Cu) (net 2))
 (segment (start 186.014 107.95) (end 186.014 109.306) (width 0.25) (layer F.Cu) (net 2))
 (segment (start 186.014 109.306) (end 186.014 110.49) (width 0.25) (layer F.Cu) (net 2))
 (segment (start 186.014 105.369) (end 186.055 105.41) (width 0.25) (layer F.Cu) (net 2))
 (segment (start 198.841 104.181) (end 200.152 102.87) (width 0.25) (layer F.Cu) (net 2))
 (segment (start 186.014 104.181) (end 198.841 104.181) (width 0.25) (layer F.Cu) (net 2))
 (segment (start 186.014 102.87) (end 186.014 104.181) (width 0.25) (layer F.Cu) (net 2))
 (segment (start 186.014 104.181) (end 186.014 105.369) (width 0.25) (layer F.Cu) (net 2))
 (segment (start 186.014 102.87) (end 184.2135 102.87) (width 0.4) (layer F.Cu) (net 2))
 (segment (start 183.896 102.5525) (end 183.896 102.489) (width 0.4) (layer F.Cu) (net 2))
 (segment (start 184.2135 102.87) (end 183.896 102.5525) (width 0.4) (layer F.Cu) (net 2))
 (segment (start 198.901999 109.200001) (end 200.152 107.95) (width 0.35) (layer F.Cu) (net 2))
 (segment (start 197.060499 109.200001) (end 198.901999 109.200001) (width 0.35) (layer F.Cu) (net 2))
 (segment (start 196.9545 109.306) (end 197.060499 109.200001) (width 0.35) (layer F.Cu) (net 2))
 (segment (start 186.014 109.306) (end 196.9545 109.306) (width 0.35) (layer F.Cu) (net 2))
 (segment (start 186.117 85.217) (end 182.324 89.01) (width 0.35) (layer B.Cu) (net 2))
 (segment (start 190.5 85.217) (end 186.117 85.217) (width 0.35) (layer B.Cu) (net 2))
 (segment (start 186.117 83.803) (end 186.117 85.217) (width 0.35) (layer B.Cu) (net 2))
 (segment (start 182.324 80.01) (end 186.117 83.803) (width 0.35) (layer B.Cu) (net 2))
 (segment (start 186.117 94.217) (end 186.117 85.217) (width 0.35) (layer B.Cu) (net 2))
 (segment (start 182.324 98.01) (end 186.117 94.217) (width 0.35) (layer B.Cu) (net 2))
 (segment (start 183.586501 99.272501) (end 183.586501 101.616001) (width 0.35) (layer B.Cu) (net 2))
 (segment (start 182.324 98.01) (end 183.586501 99.272501) (width 0.35) (layer B.Cu) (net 2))
 (via (at 183.896 102.5525) (size 0.7) (drill 0.5) (layers F.Cu B.Cu) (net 2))
 (segment (start 183.586501 102.243001) (end 183.896 102.5525) (width 0.35) (layer B.Cu) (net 2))
 (segment (start 183.586501 101.616001) (end 183.586501 102.243001) (width 0.35) (layer B.Cu) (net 2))
 (segment (start 179.324 86.01) (end 174.467 86.01) (width 0.35) (layer B.Cu) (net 2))
 (segment (start 174.467 86.01) (end 173.1645 87.3125) (width 0.35) (layer B.Cu) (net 2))
 (segment (start 173.1645 87.3125) (end 173.1645 93.726) (width 0.35) (layer B.Cu) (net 2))
 (segment (start 174.4485 95.01) (end 179.324 95.01) (width 0.35) (layer B.Cu) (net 2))
 (segment (start 173.1645 93.726) (end 174.4485 95.01) (width 0.35) (layer B.Cu) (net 2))
 (segment (start 174.3075 102.5525) (end 182.650002 102.5525) (width 0.35) (layer B.Cu) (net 2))
 (segment (start 173.1645 101.4095) (end 174.3075 102.5525) (width 0.35) (layer B.Cu) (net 2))
 (segment (start 173.1645 96.139) (end 173.1645 101.4095) (width 0.35) (layer B.Cu) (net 2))
 (segment (start 174.2935 95.01) (end 173.1645 96.139) (width 0.35) (layer B.Cu) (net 2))
 (segment (start 182.650002 102.5525) (end 183.586501 101.616001) (width 0.35) (layer B.Cu) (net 2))
 (segment (start 174.4485 95.01) (end 174.2935 95.01) (width 0.35) (layer B.Cu) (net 2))
 (segment (start 197.612 102.87) (end 192.743 102.87) (width 0.25) (layer F.Cu) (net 34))
 (segment (start 192.786 105.41) (end 197.612 105.41) (width 0.25) (layer F.Cu) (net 35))
 (segment (start 197.612 107.95) (end 192.827 107.95) (width 0.25) (layer F.Cu) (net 37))
 (segment (start 192.913 110.49) (end 197.612 110.49) (width 0.25) (layer F.Cu) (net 38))
 (segment (start 197.612 113.03) (end 192.913 113.03) (width 0.25) (layer F.Cu) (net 40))
 (segment (start 190.713 113.03) (end 188.214 113.03) (width 0.25) (layer F.Cu) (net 1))
 (segment (start 188.214 110.49) (end 190.713 110.49) (width 0.25) (layer F.Cu) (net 3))
 (segment (start 190.627 107.95) (end 188.214 107.95) (width 0.25) (layer F.Cu) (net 4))
 (segment (start 188.255 105.41) (end 190.586 105.41) (width 0.25) (layer F.Cu) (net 5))
 (segment (start 190.543 102.87) (end 188.214 102.87) (width 0.25) (layer F.Cu) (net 6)))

